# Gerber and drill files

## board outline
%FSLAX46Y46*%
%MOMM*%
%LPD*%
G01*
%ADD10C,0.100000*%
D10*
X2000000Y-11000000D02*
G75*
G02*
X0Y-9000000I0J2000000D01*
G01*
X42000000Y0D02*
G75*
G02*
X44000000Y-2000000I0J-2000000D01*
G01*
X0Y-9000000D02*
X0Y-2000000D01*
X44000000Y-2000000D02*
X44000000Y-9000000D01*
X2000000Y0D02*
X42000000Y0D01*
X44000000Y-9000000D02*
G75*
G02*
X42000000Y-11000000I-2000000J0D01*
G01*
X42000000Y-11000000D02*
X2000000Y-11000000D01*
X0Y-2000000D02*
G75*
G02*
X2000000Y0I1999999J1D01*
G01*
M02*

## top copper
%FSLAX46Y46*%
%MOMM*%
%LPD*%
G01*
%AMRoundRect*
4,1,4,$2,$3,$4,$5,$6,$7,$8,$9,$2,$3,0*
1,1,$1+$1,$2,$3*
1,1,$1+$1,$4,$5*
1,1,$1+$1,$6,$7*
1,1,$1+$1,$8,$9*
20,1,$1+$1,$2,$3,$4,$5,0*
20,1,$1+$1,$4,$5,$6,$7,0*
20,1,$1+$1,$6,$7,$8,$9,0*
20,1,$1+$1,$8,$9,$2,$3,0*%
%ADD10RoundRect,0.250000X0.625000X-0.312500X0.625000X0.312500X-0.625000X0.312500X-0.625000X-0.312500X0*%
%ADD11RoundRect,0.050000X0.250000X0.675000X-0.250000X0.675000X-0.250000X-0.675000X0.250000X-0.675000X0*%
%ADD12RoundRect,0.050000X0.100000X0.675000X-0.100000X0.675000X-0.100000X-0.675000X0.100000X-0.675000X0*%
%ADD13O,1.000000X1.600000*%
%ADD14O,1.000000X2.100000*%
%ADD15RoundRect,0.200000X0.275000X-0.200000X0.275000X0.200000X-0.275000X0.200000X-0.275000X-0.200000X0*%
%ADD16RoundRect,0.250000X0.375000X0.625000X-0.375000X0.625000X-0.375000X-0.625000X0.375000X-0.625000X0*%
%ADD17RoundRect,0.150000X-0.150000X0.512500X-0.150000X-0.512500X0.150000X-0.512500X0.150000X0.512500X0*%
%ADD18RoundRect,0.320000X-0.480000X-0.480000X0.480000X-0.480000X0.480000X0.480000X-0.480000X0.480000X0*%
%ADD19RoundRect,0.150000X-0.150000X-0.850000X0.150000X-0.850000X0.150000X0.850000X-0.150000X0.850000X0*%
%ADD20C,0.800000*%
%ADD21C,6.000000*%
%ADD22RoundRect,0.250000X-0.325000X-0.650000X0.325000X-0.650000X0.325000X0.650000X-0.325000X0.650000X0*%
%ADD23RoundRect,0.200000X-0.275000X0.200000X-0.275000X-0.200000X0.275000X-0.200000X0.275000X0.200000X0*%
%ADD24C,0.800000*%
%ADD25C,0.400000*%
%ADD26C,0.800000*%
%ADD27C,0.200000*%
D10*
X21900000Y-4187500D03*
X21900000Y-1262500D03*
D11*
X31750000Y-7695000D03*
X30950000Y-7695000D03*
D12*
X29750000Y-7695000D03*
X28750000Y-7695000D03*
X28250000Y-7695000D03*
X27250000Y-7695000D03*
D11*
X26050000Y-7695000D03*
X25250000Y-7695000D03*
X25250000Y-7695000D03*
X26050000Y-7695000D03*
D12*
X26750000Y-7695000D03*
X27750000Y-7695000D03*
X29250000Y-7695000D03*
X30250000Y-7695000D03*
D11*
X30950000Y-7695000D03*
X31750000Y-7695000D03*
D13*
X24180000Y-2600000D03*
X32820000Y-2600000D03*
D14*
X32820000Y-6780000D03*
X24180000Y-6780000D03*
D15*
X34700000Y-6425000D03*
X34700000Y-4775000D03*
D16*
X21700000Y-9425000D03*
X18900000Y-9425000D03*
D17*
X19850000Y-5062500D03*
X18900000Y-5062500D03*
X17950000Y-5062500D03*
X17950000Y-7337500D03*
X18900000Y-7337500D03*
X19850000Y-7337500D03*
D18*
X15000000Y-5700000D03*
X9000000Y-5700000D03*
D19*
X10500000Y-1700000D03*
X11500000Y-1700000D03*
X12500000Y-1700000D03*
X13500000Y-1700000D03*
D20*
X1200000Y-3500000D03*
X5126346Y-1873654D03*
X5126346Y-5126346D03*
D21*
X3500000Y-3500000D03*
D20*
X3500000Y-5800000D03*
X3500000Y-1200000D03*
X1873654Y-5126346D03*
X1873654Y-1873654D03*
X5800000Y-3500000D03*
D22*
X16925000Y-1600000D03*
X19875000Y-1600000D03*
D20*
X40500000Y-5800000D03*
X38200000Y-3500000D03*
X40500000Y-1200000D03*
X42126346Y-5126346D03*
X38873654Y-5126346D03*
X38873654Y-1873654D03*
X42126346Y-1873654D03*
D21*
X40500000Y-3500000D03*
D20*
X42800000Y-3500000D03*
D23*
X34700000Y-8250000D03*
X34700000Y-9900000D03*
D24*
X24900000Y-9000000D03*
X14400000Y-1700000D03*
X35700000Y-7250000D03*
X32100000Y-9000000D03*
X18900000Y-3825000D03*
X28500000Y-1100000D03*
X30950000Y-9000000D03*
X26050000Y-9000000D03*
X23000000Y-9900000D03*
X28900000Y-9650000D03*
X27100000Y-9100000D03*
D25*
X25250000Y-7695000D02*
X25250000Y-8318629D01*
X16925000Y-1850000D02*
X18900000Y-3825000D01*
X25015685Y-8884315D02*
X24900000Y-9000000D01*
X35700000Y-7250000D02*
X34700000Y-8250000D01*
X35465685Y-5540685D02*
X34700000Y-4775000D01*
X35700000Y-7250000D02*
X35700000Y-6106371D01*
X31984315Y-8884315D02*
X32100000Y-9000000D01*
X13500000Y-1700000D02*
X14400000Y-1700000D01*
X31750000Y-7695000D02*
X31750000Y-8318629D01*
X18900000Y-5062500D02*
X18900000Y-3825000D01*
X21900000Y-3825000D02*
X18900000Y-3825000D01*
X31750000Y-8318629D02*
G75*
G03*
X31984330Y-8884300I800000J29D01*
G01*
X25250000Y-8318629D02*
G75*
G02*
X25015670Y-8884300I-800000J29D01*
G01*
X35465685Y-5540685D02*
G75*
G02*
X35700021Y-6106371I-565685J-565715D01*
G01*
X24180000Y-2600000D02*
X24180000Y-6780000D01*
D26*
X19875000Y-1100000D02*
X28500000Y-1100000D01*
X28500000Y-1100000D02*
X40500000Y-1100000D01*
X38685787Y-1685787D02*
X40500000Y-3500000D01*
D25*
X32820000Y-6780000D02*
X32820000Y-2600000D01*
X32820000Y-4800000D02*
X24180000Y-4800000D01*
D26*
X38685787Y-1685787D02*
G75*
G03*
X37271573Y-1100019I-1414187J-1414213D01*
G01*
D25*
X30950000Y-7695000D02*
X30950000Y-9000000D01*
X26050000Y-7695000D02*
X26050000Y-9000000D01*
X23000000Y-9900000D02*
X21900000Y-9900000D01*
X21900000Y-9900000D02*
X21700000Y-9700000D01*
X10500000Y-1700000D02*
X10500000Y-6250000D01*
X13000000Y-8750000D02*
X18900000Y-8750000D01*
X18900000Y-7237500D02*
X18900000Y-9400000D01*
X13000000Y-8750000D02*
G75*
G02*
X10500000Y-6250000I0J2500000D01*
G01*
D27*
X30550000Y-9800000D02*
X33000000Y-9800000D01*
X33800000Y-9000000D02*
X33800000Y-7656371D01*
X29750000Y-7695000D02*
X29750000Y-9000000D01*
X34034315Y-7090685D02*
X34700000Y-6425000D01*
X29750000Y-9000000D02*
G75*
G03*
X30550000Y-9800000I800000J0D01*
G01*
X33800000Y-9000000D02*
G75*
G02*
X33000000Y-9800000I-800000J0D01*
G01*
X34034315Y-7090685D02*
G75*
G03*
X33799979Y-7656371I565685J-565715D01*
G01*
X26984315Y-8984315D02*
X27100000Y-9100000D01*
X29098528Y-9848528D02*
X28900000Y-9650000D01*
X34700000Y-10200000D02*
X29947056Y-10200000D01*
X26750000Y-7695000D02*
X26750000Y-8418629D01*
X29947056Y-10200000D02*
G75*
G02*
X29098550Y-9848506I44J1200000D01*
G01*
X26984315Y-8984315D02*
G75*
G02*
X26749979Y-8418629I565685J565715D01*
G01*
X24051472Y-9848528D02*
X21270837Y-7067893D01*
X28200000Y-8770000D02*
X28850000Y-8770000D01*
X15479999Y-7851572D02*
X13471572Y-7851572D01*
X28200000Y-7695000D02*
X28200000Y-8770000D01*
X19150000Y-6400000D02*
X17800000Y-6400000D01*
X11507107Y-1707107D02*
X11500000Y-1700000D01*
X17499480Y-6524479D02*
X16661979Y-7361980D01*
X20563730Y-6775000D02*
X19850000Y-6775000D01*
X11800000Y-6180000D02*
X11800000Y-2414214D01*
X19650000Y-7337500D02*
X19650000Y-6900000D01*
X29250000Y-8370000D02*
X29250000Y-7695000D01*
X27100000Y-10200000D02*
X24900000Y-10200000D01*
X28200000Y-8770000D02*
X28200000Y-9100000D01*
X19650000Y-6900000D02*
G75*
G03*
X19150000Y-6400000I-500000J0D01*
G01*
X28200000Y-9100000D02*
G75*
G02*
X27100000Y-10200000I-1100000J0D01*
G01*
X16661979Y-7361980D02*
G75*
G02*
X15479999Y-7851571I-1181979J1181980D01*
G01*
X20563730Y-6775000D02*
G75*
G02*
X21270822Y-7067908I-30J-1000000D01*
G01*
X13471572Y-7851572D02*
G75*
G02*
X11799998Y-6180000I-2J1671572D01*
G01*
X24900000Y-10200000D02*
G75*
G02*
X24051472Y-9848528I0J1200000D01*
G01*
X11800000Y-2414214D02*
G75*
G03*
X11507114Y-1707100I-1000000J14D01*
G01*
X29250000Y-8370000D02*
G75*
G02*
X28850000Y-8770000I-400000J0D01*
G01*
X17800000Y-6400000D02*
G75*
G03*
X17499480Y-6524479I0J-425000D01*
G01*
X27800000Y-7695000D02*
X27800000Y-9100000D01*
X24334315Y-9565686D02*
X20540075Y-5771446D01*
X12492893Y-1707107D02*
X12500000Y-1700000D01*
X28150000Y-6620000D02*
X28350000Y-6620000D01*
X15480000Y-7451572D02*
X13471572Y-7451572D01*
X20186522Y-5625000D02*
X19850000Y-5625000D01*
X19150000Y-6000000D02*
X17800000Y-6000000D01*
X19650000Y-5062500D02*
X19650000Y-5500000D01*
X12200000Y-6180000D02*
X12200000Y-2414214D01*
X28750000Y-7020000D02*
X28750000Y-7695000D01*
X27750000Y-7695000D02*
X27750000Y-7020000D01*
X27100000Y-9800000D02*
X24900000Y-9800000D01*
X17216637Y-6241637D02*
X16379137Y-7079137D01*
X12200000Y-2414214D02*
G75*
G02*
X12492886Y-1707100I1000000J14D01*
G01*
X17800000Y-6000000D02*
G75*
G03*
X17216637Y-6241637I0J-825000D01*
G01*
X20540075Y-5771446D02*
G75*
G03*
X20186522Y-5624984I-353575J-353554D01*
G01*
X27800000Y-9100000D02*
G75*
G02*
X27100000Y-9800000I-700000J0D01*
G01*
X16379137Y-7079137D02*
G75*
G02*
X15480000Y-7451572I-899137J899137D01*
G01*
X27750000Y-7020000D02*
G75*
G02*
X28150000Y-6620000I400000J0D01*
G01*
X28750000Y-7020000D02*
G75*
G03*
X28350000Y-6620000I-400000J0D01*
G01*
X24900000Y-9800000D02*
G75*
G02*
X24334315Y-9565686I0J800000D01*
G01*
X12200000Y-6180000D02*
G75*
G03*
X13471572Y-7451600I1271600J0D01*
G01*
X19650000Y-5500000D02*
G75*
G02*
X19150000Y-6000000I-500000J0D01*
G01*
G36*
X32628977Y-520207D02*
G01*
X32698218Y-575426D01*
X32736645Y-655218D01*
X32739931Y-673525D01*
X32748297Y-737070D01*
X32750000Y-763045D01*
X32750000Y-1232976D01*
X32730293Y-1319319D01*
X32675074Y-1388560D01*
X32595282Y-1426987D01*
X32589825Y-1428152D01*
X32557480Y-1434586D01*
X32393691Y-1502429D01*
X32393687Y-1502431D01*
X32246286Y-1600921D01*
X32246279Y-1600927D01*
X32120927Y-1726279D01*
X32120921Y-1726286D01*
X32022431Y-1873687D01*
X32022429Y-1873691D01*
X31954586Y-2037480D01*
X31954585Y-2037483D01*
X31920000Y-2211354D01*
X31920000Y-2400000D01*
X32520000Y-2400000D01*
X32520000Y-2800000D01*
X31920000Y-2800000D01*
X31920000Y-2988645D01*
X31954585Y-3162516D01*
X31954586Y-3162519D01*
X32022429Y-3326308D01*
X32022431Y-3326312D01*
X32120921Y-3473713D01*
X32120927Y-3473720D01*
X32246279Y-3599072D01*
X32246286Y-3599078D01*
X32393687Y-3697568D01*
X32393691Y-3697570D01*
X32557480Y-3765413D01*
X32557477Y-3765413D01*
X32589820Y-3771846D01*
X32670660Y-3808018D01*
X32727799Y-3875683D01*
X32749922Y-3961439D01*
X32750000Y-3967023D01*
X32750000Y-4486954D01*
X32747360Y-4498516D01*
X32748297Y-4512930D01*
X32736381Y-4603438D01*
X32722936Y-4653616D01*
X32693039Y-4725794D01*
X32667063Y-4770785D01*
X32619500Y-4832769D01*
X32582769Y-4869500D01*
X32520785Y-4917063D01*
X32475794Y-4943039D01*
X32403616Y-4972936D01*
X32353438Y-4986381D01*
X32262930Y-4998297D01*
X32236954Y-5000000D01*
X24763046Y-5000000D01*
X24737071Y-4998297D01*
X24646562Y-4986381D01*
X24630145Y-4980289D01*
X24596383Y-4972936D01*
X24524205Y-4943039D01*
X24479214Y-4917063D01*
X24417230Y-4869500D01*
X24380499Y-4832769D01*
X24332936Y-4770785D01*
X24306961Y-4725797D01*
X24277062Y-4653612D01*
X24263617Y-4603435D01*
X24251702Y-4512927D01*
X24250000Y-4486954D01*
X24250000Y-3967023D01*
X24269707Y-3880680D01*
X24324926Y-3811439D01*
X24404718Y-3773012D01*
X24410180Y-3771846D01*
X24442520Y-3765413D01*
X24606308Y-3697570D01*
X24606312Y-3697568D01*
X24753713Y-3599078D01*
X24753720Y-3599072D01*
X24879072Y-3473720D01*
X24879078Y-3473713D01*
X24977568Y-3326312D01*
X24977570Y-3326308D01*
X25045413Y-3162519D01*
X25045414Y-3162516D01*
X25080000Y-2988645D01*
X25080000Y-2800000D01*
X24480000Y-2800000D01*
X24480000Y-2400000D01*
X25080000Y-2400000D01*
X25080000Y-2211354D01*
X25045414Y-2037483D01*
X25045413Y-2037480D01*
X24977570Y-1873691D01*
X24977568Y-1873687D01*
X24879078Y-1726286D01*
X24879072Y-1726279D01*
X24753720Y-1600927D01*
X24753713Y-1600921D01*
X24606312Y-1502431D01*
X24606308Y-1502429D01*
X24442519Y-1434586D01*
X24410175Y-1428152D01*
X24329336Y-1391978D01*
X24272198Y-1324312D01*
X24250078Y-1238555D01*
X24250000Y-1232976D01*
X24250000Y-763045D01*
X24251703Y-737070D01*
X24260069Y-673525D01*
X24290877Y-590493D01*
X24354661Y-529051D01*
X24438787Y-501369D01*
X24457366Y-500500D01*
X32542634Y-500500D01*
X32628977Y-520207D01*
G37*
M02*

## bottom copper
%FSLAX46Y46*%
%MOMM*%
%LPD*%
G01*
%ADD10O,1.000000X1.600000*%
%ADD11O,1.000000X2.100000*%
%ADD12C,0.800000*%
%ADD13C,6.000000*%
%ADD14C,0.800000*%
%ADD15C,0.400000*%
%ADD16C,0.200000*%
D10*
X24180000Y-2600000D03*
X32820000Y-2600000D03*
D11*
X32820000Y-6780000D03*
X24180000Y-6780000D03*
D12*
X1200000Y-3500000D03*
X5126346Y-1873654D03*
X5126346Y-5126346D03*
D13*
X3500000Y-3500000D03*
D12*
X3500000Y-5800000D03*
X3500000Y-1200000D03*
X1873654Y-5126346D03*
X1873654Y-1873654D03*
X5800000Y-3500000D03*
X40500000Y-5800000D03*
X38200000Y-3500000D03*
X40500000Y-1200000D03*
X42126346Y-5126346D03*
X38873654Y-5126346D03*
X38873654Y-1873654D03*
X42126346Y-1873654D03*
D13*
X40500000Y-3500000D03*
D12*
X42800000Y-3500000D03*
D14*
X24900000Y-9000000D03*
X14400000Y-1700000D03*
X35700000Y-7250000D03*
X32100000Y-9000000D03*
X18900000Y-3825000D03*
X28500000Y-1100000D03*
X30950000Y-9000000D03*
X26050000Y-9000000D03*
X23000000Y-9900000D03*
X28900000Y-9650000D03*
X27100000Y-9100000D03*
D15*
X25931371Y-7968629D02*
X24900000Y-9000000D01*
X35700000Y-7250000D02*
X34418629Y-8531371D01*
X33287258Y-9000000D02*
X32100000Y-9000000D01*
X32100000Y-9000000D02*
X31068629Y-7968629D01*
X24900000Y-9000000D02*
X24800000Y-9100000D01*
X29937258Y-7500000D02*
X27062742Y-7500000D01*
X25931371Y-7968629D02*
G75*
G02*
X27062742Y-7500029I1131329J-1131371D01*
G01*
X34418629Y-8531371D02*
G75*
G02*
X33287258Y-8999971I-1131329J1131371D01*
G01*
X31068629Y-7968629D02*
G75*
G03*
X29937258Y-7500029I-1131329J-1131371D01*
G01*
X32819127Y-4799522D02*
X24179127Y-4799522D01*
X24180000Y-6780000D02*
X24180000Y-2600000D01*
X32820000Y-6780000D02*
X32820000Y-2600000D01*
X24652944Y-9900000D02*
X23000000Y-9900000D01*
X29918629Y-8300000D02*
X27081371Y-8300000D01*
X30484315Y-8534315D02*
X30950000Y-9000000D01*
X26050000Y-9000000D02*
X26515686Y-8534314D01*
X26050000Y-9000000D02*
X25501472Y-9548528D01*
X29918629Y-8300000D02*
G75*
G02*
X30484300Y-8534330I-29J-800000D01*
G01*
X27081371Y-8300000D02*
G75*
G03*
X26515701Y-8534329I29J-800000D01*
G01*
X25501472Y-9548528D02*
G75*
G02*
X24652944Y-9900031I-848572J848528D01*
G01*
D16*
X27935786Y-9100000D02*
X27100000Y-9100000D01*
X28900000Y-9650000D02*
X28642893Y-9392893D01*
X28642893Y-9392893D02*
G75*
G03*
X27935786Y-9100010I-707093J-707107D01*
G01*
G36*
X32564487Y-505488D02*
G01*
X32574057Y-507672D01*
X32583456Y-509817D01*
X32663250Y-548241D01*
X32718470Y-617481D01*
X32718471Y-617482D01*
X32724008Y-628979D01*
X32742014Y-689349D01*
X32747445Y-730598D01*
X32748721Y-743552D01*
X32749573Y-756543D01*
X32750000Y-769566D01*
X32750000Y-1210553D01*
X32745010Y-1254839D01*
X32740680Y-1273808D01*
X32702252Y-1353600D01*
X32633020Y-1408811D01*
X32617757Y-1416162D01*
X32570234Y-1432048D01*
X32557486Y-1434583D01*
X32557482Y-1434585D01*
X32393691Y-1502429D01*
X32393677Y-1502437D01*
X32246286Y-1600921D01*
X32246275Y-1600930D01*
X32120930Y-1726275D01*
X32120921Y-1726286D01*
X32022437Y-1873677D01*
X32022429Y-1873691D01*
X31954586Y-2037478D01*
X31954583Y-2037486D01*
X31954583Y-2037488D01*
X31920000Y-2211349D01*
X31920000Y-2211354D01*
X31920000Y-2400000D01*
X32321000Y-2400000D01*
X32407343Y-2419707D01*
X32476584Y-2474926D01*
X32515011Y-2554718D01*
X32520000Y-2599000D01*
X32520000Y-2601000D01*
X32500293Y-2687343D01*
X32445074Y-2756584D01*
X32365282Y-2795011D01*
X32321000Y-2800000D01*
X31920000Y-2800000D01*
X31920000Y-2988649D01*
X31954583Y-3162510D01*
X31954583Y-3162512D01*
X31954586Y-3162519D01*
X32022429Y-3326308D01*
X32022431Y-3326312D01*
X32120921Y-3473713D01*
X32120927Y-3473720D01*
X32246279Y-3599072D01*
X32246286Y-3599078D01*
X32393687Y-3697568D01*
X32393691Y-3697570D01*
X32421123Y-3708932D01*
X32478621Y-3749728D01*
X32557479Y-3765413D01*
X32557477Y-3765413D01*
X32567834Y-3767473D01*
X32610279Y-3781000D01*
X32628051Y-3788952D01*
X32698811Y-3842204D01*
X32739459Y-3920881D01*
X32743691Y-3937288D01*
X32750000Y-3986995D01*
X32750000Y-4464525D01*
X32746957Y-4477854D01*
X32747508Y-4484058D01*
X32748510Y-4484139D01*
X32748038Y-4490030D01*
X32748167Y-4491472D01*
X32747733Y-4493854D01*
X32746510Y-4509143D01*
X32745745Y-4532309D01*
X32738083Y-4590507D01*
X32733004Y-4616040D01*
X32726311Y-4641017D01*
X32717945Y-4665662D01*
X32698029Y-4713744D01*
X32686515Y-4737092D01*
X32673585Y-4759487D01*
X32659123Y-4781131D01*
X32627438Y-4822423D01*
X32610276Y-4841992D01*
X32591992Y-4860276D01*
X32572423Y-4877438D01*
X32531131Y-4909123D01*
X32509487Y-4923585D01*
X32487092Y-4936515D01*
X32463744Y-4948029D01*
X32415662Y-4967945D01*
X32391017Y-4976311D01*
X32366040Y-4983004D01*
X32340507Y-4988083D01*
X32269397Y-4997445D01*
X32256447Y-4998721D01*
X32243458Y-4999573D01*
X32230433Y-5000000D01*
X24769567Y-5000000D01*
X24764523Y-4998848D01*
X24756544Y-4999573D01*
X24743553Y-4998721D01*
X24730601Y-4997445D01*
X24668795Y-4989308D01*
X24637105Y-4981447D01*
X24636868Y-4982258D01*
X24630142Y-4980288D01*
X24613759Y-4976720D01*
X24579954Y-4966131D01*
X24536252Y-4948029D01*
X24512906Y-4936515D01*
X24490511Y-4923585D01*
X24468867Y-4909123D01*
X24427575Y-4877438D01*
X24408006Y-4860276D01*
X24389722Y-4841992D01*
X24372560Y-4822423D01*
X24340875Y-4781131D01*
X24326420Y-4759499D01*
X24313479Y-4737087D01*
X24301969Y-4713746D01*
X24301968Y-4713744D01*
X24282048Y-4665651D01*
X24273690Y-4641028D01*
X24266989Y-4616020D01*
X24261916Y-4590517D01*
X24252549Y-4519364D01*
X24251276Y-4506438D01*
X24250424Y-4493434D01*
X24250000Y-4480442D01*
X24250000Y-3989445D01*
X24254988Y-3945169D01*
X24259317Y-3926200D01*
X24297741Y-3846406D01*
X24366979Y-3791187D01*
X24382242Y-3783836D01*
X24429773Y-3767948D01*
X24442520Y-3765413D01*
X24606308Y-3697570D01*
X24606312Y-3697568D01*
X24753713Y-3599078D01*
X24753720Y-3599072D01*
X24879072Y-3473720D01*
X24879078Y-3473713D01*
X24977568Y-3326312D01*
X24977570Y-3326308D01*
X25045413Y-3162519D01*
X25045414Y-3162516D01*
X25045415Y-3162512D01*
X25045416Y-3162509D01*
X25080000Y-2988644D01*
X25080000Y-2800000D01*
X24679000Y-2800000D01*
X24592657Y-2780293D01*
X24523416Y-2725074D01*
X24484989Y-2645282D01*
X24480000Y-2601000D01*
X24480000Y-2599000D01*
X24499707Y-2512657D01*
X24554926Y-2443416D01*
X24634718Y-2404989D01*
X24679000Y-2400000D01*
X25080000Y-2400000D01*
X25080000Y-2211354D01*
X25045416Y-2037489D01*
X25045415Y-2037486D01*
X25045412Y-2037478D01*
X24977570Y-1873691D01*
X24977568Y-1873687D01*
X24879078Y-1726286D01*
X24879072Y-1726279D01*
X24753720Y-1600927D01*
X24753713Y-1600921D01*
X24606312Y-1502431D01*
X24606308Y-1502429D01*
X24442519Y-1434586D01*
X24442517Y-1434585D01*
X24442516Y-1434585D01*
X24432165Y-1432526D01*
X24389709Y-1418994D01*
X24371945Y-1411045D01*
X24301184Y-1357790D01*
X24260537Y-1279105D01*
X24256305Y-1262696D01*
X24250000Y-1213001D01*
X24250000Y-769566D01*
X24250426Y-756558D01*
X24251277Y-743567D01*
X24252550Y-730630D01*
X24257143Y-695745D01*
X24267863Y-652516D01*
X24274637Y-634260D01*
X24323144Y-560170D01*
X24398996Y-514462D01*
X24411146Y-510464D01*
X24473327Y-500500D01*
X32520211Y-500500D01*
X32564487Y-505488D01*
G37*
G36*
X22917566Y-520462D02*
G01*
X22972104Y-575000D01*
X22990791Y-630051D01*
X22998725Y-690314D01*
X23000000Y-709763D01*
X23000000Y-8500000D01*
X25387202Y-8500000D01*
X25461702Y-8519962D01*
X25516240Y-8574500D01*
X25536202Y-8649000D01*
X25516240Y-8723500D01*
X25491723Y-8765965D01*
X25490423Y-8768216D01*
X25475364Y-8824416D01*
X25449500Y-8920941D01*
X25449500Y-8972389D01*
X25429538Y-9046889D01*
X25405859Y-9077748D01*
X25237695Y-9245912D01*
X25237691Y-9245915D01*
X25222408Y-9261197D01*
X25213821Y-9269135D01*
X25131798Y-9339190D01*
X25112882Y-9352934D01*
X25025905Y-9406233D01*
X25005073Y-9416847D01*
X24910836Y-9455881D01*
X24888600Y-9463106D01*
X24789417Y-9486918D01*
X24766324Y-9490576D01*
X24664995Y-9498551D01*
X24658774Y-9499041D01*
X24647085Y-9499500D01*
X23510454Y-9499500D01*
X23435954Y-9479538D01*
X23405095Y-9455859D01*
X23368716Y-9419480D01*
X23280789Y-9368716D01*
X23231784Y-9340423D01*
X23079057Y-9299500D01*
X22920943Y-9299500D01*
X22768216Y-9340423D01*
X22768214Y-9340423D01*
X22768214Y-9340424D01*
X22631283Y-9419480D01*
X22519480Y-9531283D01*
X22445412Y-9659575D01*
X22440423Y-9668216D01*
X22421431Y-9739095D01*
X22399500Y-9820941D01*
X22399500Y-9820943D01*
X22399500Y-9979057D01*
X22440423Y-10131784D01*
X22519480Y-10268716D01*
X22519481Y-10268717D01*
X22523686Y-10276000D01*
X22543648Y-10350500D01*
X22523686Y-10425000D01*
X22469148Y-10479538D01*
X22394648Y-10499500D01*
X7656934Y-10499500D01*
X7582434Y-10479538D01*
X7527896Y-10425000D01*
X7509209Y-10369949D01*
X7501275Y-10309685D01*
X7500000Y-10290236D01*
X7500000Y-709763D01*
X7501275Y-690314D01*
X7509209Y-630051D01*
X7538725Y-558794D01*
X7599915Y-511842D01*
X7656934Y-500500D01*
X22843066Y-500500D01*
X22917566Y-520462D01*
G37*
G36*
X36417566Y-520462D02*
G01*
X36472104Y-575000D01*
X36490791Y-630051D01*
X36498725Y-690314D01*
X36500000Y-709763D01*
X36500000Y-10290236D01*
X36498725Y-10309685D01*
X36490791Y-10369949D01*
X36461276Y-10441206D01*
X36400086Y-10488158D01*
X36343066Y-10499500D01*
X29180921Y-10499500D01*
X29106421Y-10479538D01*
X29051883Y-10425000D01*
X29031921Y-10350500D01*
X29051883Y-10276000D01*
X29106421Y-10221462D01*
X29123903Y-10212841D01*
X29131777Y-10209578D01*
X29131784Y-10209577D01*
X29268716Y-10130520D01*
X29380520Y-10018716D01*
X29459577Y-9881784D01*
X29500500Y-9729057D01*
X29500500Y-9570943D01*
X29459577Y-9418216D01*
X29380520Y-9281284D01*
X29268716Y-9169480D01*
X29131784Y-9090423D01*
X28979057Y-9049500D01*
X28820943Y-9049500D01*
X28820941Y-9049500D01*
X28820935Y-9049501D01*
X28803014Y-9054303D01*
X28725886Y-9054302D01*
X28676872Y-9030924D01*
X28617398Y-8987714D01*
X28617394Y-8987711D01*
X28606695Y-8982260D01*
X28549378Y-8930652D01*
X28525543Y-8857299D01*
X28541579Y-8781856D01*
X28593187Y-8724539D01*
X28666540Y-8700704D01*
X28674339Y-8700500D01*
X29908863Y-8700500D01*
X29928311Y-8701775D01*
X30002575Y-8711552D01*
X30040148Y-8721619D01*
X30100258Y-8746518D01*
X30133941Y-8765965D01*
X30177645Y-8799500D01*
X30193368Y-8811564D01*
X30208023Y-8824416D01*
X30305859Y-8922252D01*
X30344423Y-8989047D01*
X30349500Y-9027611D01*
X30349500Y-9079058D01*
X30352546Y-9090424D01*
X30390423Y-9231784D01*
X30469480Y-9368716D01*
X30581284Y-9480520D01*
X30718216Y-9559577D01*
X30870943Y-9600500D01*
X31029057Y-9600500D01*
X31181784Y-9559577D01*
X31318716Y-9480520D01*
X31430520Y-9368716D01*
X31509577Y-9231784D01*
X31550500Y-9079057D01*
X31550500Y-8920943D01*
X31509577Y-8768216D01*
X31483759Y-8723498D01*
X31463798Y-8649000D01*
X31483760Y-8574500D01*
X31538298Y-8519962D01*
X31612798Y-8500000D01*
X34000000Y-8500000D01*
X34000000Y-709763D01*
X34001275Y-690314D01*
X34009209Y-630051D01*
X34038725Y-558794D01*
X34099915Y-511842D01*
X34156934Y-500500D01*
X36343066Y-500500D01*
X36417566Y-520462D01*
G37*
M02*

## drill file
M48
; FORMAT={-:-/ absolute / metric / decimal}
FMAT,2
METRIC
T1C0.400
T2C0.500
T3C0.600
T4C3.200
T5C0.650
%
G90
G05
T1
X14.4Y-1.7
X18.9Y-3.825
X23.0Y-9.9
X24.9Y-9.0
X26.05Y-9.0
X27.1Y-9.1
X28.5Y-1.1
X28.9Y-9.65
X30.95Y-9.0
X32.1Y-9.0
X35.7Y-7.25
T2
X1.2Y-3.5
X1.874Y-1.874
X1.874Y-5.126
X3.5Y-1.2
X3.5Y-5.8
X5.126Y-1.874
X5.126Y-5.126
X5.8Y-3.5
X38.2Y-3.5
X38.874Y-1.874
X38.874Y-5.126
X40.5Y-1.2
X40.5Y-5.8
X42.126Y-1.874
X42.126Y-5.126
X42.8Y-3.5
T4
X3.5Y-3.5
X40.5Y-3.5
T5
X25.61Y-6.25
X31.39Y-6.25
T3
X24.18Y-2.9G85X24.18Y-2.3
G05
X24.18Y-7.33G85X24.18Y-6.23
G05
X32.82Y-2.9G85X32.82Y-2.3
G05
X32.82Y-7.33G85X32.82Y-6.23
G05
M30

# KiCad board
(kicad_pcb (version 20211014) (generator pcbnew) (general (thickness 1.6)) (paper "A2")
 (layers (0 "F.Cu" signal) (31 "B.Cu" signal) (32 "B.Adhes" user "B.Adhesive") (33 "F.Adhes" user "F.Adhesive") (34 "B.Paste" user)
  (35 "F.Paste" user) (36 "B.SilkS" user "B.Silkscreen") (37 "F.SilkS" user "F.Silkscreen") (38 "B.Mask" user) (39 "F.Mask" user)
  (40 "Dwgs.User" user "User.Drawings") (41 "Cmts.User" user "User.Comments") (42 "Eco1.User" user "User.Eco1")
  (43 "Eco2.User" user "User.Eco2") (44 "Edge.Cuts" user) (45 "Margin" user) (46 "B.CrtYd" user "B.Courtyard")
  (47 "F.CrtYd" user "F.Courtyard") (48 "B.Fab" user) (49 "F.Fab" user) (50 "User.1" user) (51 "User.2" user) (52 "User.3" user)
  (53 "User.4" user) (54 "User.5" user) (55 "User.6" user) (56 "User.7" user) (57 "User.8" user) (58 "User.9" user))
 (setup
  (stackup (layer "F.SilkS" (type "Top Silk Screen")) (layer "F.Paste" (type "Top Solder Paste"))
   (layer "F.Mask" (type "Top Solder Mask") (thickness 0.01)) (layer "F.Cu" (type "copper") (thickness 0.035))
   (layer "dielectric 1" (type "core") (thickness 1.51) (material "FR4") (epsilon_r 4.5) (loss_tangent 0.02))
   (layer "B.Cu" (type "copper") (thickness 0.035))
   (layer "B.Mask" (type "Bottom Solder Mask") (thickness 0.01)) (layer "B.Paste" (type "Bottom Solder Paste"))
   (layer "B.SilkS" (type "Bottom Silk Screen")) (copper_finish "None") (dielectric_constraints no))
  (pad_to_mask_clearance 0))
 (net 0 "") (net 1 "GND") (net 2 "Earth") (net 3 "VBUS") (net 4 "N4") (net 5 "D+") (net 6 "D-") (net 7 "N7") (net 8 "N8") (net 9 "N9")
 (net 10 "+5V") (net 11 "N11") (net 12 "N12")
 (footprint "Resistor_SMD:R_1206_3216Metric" (layer "F.Cu") (at 21.9 2.725 90)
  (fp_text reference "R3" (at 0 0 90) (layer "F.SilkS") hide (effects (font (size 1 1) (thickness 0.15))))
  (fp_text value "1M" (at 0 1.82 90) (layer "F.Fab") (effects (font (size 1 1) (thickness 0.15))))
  (pad "1" smd roundrect (at -1.4625 0 90) (size 1.125 1.75) (layers "F.Cu" "F.Paste" "F.Mask") (roundrect_rratio 0.2222222222)
   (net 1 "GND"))
  (pad "2" smd roundrect (at 1.4625 0 90) (size 1.125 1.75) (layers "F.Cu" "F.Paste" "F.Mask") (roundrect_rratio 0.2222222222)
   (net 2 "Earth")))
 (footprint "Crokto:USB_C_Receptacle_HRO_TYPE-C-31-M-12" (layer "F.Cu") (at 28.5 3.65 180)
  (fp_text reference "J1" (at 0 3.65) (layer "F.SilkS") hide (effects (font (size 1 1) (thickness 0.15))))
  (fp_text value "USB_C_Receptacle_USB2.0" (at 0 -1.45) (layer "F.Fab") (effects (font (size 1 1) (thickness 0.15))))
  (pad "" np_thru_hole circle (at -2.89 -2.6 180) (size 0.65 0.65) (drill 0.65) (layers *.Cu *.Mask))
  (pad "" np_thru_hole circle (at 2.89 -2.6 180) (size 0.65 0.65) (drill 0.65) (layers *.Cu *.Mask))
  (pad "A1" smd roundrect (at -3.25 -4.045 180) (size 0.6 1.45) (layers "F.Cu" "F.Paste" "F.Mask") (roundrect_rratio 0.08333333333)
   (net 1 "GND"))
  (pad "A4" smd roundrect (at -2.45 -4.045 180) (size 0.6 1.45) (layers "F.Cu" "F.Paste" "F.Mask") (roundrect_rratio 0.08333333333)
   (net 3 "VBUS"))
  (pad "A5" smd roundrect (at -1.25 -4.045 180) (size 0.3 1.45) (layers "F.Cu" "F.Paste" "F.Mask") (roundrect_rratio 0.1666666667)
   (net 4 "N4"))
  (pad "A6" smd roundrect (at -0.25 -4.045 180) (size 0.3 1.45) (layers "F.Cu" "F.Paste" "F.Mask") (roundrect_rratio 0.1666666667)
   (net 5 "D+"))
  (pad "A7" smd roundrect (at 0.25 -4.045 180) (size 0.3 1.45) (layers "F.Cu" "F.Paste" "F.Mask") (roundrect_rratio 0.1666666667)
   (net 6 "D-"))
  (pad "A8" smd roundrect (at 1.25 -4.045 180) (size 0.3 1.45) (layers "F.Cu" "F.Paste" "F.Mask") (roundrect_rratio 0.1666666667)
   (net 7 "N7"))
  (pad "A9" smd roundrect (at 2.45 -4.045 180) (size 0.6 1.45) (layers "F.Cu" "F.Paste" "F.Mask") (roundrect_rratio 0.08333333333)
   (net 3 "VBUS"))
  (pad "A12" smd roundrect (at 3.25 -4.045 180) (size 0.6 1.45) (layers "F.Cu" "F.Paste" "F.Mask") (roundrect_rratio 0.08333333333)
   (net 1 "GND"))
  (pad "B1" smd roundrect (at 3.25 -4.045 180) (size 0.6 1.45) (layers "F.Cu" "F.Paste" "F.Mask") (roundrect_rratio 0.08333333333)
   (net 1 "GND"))
  (pad "B4" smd roundrect (at 2.45 -4.045 180) (size 0.6 1.45) (layers "F.Cu" "F.Paste" "F.Mask") (roundrect_rratio 0.08333333333)
   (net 3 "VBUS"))
  (pad "B5" smd roundrect (at 1.75 -4.045 180) (size 0.3 1.45) (layers "F.Cu" "F.Paste" "F.Mask") (roundrect_rratio 0.1666666667)
   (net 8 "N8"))
  (pad "B6" smd roundrect (at 0.75 -4.045 180) (size 0.3 1.45) (layers "F.Cu" "F.Paste" "F.Mask") (roundrect_rratio 0.1666666667)
   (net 5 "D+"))
  (pad "B7" smd roundrect (at -0.75 -4.045 180) (size 0.3 1.45) (layers "F.Cu" "F.Paste" "F.Mask") (roundrect_rratio 0.1666666667)
   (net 6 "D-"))
  (pad "B8" smd roundrect (at -1.75 -4.045 180) (size 0.3 1.45) (layers "F.Cu" "F.Paste" "F.Mask") (roundrect_rratio 0.1666666667)
   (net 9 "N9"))
  (pad "B9" smd roundrect (at -2.45 -4.045 180) (size 0.6 1.45) (layers "F.Cu" "F.Paste" "F.Mask") (roundrect_rratio 0.08333333333)
   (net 3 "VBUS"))
  (pad "B12" smd roundrect (at -3.25 -4.045 180) (size 0.6 1.45) (layers "F.Cu" "F.Paste" "F.Mask") (roundrect_rratio 0.08333333333)
   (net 1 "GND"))
  (pad "S1" thru_hole oval (at 4.32 1.05 180) (size 1 1.6) (drill oval 0.6 1.2) (layers *.Cu *.Mask) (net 2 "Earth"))
  (pad "S1" thru_hole oval (at -4.32 1.05 180) (size 1 1.6) (drill oval 0.6 1.2) (layers *.Cu *.Mask) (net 2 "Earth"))
  (pad "S1" thru_hole oval (at -4.32 -3.13 180) (size 1 2.1) (drill oval 0.6 1.7) (layers *.Cu *.Mask) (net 2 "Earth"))
  (pad "S1" thru_hole oval (at 4.32 -3.13 180) (size 1 2.1) (drill oval 0.6 1.7) (layers *.Cu *.Mask) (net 2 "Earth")))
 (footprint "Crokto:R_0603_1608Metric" (layer "F.Cu") (at 34.7 5.6 90)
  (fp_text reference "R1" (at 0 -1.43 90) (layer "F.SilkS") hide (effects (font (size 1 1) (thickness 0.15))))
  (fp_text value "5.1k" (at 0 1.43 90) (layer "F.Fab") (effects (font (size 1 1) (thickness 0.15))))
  (pad "1" smd roundrect (at -0.825 0 90) (size 0.8 0.95) (layers "F.Cu" "F.Paste" "F.Mask") (roundrect_rratio 0.25) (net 4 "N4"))
  (pad "2" smd roundrect (at 0.825 0 90) (size 0.8 0.95) (layers "F.Cu" "F.Paste" "F.Mask") (roundrect_rratio 0.25) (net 1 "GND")))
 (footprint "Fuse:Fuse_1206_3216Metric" (layer "F.Cu") (at 20.3 9.425 180)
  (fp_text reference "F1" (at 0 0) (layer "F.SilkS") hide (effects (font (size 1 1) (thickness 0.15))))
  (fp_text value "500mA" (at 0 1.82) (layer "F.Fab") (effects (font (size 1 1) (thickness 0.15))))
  (pad "1" smd roundrect (at -1.4 0 180) (size 1.25 1.75) (layers "F.Cu" "F.Paste" "F.Mask") (roundrect_rratio 0.2) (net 3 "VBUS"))
  (pad "2" smd roundrect (at 1.4 0 180) (size 1.25 1.75) (layers "F.Cu" "F.Paste" "F.Mask") (roundrect_rratio 0.2) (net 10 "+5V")))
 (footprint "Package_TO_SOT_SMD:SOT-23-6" (layer "F.Cu") (at 18.9 6.2 -90)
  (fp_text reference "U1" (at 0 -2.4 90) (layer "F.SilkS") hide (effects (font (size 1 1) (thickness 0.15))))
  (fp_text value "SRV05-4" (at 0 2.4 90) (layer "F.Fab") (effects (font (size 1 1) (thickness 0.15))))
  (pad "1" smd roundrect (at -1.1375 -0.95 270) (size 1.325 0.6) (layers "F.Cu" "F.Paste" "F.Mask") (roundrect_rratio 0.25) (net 5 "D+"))
  (pad "2" smd roundrect (at -1.1375 0 270) (size 1.325 0.6) (layers "F.Cu" "F.Paste" "F.Mask") (roundrect_rratio 0.25) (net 1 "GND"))
  (pad "3" smd roundrect (at -1.1375 0.95 270) (size 1.325 0.6) (layers "F.Cu" "F.Paste" "F.Mask") (roundrect_rratio 0.25) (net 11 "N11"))
  (pad "4" smd roundrect (at 1.1375 0.95 270) (size 1.325 0.6) (layers "F.Cu" "F.Paste" "F.Mask") (roundrect_rratio 0.25) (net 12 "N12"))
  (pad "5" smd roundrect (at 1.1375 0 270) (size 1.325 0.6) (layers "F.Cu" "F.Paste" "F.Mask") (roundrect_rratio 0.25) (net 10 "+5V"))
  (pad "6" smd roundrect (at 1.1375 -0.95 270) (size 1.325 0.6) (layers "F.Cu" "F.Paste" "F.Mask") (roundrect_rratio 0.25) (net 6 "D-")))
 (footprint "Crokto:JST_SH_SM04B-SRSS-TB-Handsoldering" (layer "F.Cu") (at 12 3.925)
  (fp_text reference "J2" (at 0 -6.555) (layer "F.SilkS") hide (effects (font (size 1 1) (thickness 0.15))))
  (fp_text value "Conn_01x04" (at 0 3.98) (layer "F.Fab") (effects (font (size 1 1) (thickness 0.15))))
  (pad "" smd roundrect (at 3 1.775) (size 1.6 1.6) (layers "F.Cu" "F.Paste" "F.Mask") (roundrect_rratio 0.2))
  (pad "" smd roundrect (at -3 1.775) (size 1.6 1.6) (layers "F.Cu" "F.Paste" "F.Mask") (roundrect_rratio 0.2))
  (pad "1" smd roundrect (at -1.5 -2.225) (size 0.6 2) (layers "F.Cu" "F.Paste" "F.Mask") (roundrect_rratio 0.25) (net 10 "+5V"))
  (pad "2" smd roundrect (at -0.5 -2.225) (size 0.6 2) (layers "F.Cu" "F.Paste" "F.Mask") (roundrect_rratio 0.25) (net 6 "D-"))
  (pad "3" smd roundrect (at 0.5 -2.225) (size 0.6 2) (layers "F.Cu" "F.Paste" "F.Mask") (roundrect_rratio 0.25) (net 5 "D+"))
  (pad "4" smd roundrect (at 1.5 -2.225) (size 0.6 2) (layers "F.Cu" "F.Paste" "F.Mask") (roundrect_rratio 0.25) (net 1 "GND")))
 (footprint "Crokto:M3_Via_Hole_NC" (layer "F.Cu") (at 3.5 3.5)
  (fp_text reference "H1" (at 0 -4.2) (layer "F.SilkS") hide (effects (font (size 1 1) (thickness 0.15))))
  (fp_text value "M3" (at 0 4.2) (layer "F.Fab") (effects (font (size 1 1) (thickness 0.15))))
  (pad "" thru_hole circle (at -2.3 0) (size 0.8 0.8) (drill 0.5) (layers *.Cu "F.Mask"))
  (pad "" thru_hole circle (at 1.626346 -1.626346) (size 0.8 0.8) (drill 0.5) (layers *.Cu "F.Mask"))
  (pad "" thru_hole circle (at 1.626346 1.626346) (size 0.8 0.8) (drill 0.5) (layers *.Cu "F.Mask"))
  (pad "" thru_hole circle (at 0 0) (size 6 6) (drill 3.2) (layers *.Cu "F.Mask"))
  (pad "" thru_hole circle (at 0 2.3) (size 0.8 0.8) (drill 0.5) (layers *.Cu "F.Mask"))
  (pad "" thru_hole circle (at 0 -2.3) (size 0.8 0.8) (drill 0.5) (layers *.Cu "F.Mask"))
  (pad "" thru_hole circle (at -1.626346 1.626346) (size 0.8 0.8) (drill 0.5) (layers *.Cu "F.Mask"))
  (pad "" thru_hole circle (at -1.626346 -1.626346) (size 0.8 0.8) (drill 0.5) (layers *.Cu "F.Mask"))
  (pad "" thru_hole circle (at 2.3 0) (size 0.8 0.8) (drill 0.5) (layers *.Cu "F.Mask")))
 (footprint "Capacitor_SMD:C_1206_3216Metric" (layer "F.Cu") (at 18.4 1.6)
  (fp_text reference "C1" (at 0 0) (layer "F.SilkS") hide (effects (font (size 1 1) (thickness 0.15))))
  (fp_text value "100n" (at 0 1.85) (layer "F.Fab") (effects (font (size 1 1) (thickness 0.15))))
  (pad "1" smd roundrect (at -1.475 0) (size 1.15 1.8) (layers "F.Cu" "F.Paste" "F.Mask") (roundrect_rratio 0.2173913043) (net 1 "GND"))
  (pad "2" smd roundrect (at 1.475 0) (size 1.15 1.8) (layers "F.Cu" "F.Paste" "F.Mask") (roundrect_rratio 0.2173913043) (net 2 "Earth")))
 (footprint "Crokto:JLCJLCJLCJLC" (layer "F.Cu") (at 28.5 4.6 180)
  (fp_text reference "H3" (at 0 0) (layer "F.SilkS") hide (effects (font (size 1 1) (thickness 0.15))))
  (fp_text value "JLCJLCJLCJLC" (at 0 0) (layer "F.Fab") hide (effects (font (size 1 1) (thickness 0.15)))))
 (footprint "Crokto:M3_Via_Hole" (layer "F.Cu") (at 40.5 3.5)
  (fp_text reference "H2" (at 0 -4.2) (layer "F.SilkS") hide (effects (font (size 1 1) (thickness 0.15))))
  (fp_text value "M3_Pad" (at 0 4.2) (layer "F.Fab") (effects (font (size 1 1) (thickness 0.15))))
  (pad "1" thru_hole circle locked (at 0 2.3) (size 0.8 0.8) (drill 0.5) (layers *.Cu *.Mask) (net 2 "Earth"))
  (pad "1" thru_hole circle locked (at -2.3 0) (size 0.8 0.8) (drill 0.5) (layers *.Cu *.Mask) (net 2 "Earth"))
  (pad "1" thru_hole circle locked (at 0 -2.3) (size 0.8 0.8) (drill 0.5) (layers *.Cu *.Mask) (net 2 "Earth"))
  (pad "1" thru_hole circle locked (at 1.626346 1.626346) (size 0.8 0.8) (drill 0.5) (layers *.Cu *.Mask) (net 2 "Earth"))
  (pad "1" thru_hole circle locked (at -1.626346 1.626346) (size 0.8 0.8) (drill 0.5) (layers *.Cu *.Mask) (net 2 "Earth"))
  (pad "1" thru_hole circle locked (at -1.626346 -1.626346) (size 0.8 0.8) (drill 0.5) (layers *.Cu *.Mask) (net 2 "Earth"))
  (pad "1" thru_hole circle locked (at 1.626346 -1.626346) (size 0.8 0.8) (drill 0.5) (layers *.Cu *.Mask) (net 2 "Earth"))
  (pad "1" thru_hole circle locked (at 0 0) (size 6 6) (drill 3.2) (layers *.Cu *.Mask) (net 2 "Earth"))
  (pad "1" thru_hole circle locked (at 2.3 0) (size 0.8 0.8) (drill 0.5) (layers *.Cu *.Mask) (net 2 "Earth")))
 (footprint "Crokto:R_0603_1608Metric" (layer "F.Cu") (at 34.7 9.075 -90)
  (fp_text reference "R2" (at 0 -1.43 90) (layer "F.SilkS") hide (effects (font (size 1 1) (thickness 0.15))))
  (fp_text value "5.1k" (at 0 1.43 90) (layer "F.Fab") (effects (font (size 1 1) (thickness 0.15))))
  (pad "1" smd roundrect (at -0.825 0 270) (size 0.8 0.95) (layers "F.Cu" "F.Paste" "F.Mask") (roundrect_rratio 0.25) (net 1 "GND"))
  (pad "2" smd roundrect (at 0.825 0 270) (size 0.8 0.95) (layers "F.Cu" "F.Paste" "F.Mask") (roundrect_rratio 0.25) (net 8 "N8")))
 (gr_arc (start 2 11) (mid 0.585786 10.414214) (end 0 9) (layer "Edge.Cuts") (width 0.1))
 (gr_arc (start 42 0) (mid 43.414214 0.585786) (end 44 2) (layer "Edge.Cuts") (width 0.1))
 (gr_line (start 0 9) (end 0 2) (layer "Edge.Cuts") (width 0.1))
 (gr_line (start 44 2) (end 44 9) (layer "Edge.Cuts") (width 0.1))
 (gr_line (start 2 0) (end 42 0) (layer "Edge.Cuts") (width 0.1))
 (gr_arc (start 44 9) (mid 43.414214 10.414214) (end 42 11) (layer "Edge.Cuts") (width 0.1))
 (gr_line (start 42 11) (end 2 11) (layer "Edge.Cuts") (width 0.1))
 (gr_arc (start 0 2) (mid 0.585786 0.585786) (end 2 0) (layer "Edge.Cuts") (width 0.1))
 (segment (start 25.25 7.695) (end 25.25 8.318629) (width 0.4) (layer "F.Cu") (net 1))
 (segment (start 16.925 1.85) (end 18.9 3.825) (width 0.4) (layer "F.Cu") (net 1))
 (segment (start 25.015685 8.884315) (end 24.9 9) (width 0.4) (layer "F.Cu") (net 1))
 (segment (start 35.7 7.25) (end 34.7 8.25) (width 0.4) (layer "F.Cu") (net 1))
 (segment (start 35.465685 5.540685) (end 34.7 4.775) (width 0.4) (layer "F.Cu") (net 1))
 (segment (start 35.7 7.25) (end 35.7 6.106371) (width 0.4) (layer "F.Cu") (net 1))
 (segment (start 31.984315 8.884315) (end 32.1 9) (width 0.4) (layer "F.Cu") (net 1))
 (segment (start 13.5 1.7) (end 14.4 1.7) (width 0.4) (layer "F.Cu") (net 1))
 (segment (start 31.75 7.695) (end 31.75 8.318629) (width 0.4) (layer "F.Cu") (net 1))
 (segment (start 18.9 5.0625) (end 18.9 3.825) (width 0.4) (layer "F.Cu") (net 1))
 (segment (start 21.9 3.825) (end 18.9 3.825) (width 0.4) (layer "F.Cu") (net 1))
 (via (at 24.9 9) (size 0.8) (drill 0.4) (layers "F.Cu" "B.Cu") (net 1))
 (via (at 14.4 1.7) (size 0.8) (drill 0.4) (layers "F.Cu" "B.Cu") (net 1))
 (via (at 35.7 7.25) (size 0.8) (drill 0.4) (layers "F.Cu" "B.Cu") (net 1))
 (via (at 32.1 9) (size 0.8) (drill 0.4) (layers "F.Cu" "B.Cu") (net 1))
 (via (at 18.9 3.825) (size 0.8) (drill 0.4) (layers "F.Cu" "B.Cu") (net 1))
 (arc (start 31.75 8.318629) (mid 31.810897 8.624776) (end 31.984315 8.884315) (width 0.4) (layer "F.Cu") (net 1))
 (arc (start 25.25 8.318629) (mid 25.189103 8.624776) (end 25.015685 8.884315) (width 0.4) (layer "F.Cu") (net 1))
 (arc (start 35.465685 5.540685) (mid 35.639104 5.800224) (end 35.7 6.106371) (width 0.4) (layer "F.Cu") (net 1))
 (segment (start 25.931371 7.968629) (end 24.9 9) (width 0.4) (layer "B.Cu") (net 1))
 (segment (start 35.7 7.25) (end 34.418629 8.531371) (width 0.4) (layer "B.Cu") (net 1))
 (segment (start 33.287258 9) (end 32.1 9) (width 0.4) (layer "B.Cu") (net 1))
 (segment (start 32.1 9) (end 31.068629 7.968629) (width 0.4) (layer "B.Cu") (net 1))
 (segment (start 24.9 9) (end 24.8 9.1) (width 0.4) (layer "B.Cu") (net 1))
 (segment (start 29.937258 7.5) (end 27.062742 7.5) (width 0.4) (layer "B.Cu") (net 1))
 (arc (start 25.931371 7.968629) (mid 26.450448 7.621793) (end 27.062742 7.5) (width 0.4) (layer "B.Cu") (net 1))
 (arc (start 34.418629 8.531371) (mid 33.899552 8.878207) (end 33.287258 9) (width 0.4) (layer "B.Cu") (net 1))
 (arc (start 31.068629 7.968629) (mid 30.549552 7.621793) (end 29.937258 7.5) (width 0.4) (layer "B.Cu") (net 1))
 (segment (start 24.18 2.6) (end 24.18 6.78) (width 0.4) (layer "F.Cu") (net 2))
 (segment (start 19.875 1.1) (end 28.5 1.1) (width 0.8) (layer "F.Cu") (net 2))
 (segment (start 28.5 1.1) (end 40.5 1.1) (width 0.8) (layer "F.Cu") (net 2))
 (segment (start 38.685787 1.685787) (end 40.5 3.5) (width 0.8) (layer "F.Cu") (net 2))
 (segment (start 32.82 6.78) (end 32.82 2.6) (width 0.4) (layer "F.Cu") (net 2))
 (segment (start 32.82 4.8) (end 24.18 4.8) (width 0.4) (layer "F.Cu") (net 2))
 (via (at 28.5 1.1) (size 0.8) (drill 0.4) (layers "F.Cu" "B.Cu") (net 2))
 (arc (start 38.685787 1.685787) (mid 38.03694 1.252241) (end 37.271573 1.1) (width 0.8) (layer "F.Cu") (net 2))
 (segment (start 32.819127 4.799522) (end 24.179127 4.799522) (width 0.4) (layer "B.Cu") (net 2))
 (segment (start 24.18 6.78) (end 24.18 2.6) (width 0.4) (layer "B.Cu") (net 2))
 (segment (start 32.82 6.78) (end 32.82 2.6) (width 0.4) (layer "B.Cu") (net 2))
 (segment (start 30.95 7.695) (end 30.95 9) (width 0.4) (layer "F.Cu") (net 3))
 (segment (start 26.05 7.695) (end 26.05 9) (width 0.4) (layer "F.Cu") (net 3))
 (segment (start 23 9.9) (end 21.9 9.9) (width 0.4) (layer "F.Cu") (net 3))
 (segment (start 21.9 9.9) (end 21.7 9.7) (width 0.4) (layer "F.Cu") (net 3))
 (via (at 30.95 9) (size 0.8) (drill 0.4) (layers "F.Cu" "B.Cu") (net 3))
 (via (at 26.05 9) (size 0.8) (drill 0.4) (layers "F.Cu" "B.Cu") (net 3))
 (via (at 23 9.9) (size 0.8) (drill 0.4) (layers "F.Cu" "B.Cu") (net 3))
 (segment (start 24.652944 9.9) (end 23 9.9) (width 0.4) (layer "B.Cu") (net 3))
 (segment (start 29.918629 8.3) (end 27.081371 8.3) (width 0.4) (layer "B.Cu") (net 3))
 (segment (start 30.484315 8.534315) (end 30.95 9) (width 0.4) (layer "B.Cu") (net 3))
 (segment (start 26.05 9) (end 26.515686 8.534314) (width 0.4) (layer "B.Cu") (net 3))
 (segment (start 26.05 9) (end 25.501472 9.548528) (width 0.4) (layer "B.Cu") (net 3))
 (arc (start 29.918629 8.3) (mid 30.224776 8.360897) (end 30.484315 8.534315) (width 0.4) (layer "B.Cu") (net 3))
 (arc (start 27.081371 8.3) (mid 26.775225 8.360896) (end 26.515686 8.534314) (width 0.4) (layer "B.Cu") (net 3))
 (arc (start 25.501472 9.548528) (mid 25.112164 9.808655) (end 24.652944 9.9) (width 0.4) (layer "B.Cu") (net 3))
 (segment (start 10.5 1.7) (end 10.5 6.25) (width 0.4) (layer "F.Cu") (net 10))
 (segment (start 13 8.75) (end 18.9 8.75) (width 0.4) (layer "F.Cu") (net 10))
 (segment (start 18.9 7.2375) (end 18.9 9.4) (width 0.4) (layer "F.Cu") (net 10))
 (arc (start 13 8.75) (mid 11.232233 8.017767) (end 10.5 6.25) (width 0.4) (layer "F.Cu") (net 10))
 (segment (start 30.55 9.8) (end 33 9.8) (width 0.2) (layer "F.Cu") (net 4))
 (segment (start 33.8 9) (end 33.8 7.656371) (width 0.2) (layer "F.Cu") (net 4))
 (segment (start 29.75 7.695) (end 29.75 9) (width 0.2) (layer "F.Cu") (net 4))
 (segment (start 34.034315 7.090685) (end 34.7 6.425) (width 0.2) (layer "F.Cu") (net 4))
 (arc (start 29.75 9) (mid 29.984315 9.565685) (end 30.55 9.8) (width 0.2) (layer "F.Cu") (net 4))
 (arc (start 33.8 9) (mid 33.565685 9.565685) (end 33 9.8) (width 0.2) (layer "F.Cu") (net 4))
 (arc (start 34.034315 7.090685) (mid 33.860896 7.350224) (end 33.8 7.656371) (width 0.2) (layer "F.Cu") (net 4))
 (segment (start 26.984315 8.984315) (end 27.1 9.1) (width 0.2) (layer "F.Cu") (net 8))
 (segment (start 29.098528 9.848528) (end 28.9 9.65) (width 0.2) (layer "F.Cu") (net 8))
 (segment (start 34.7 10.2) (end 29.947056 10.2) (width 0.2) (layer "F.Cu") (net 8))
 (segment (start 26.75 7.695) (end 26.75 8.418629) (width 0.2) (layer "F.Cu") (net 8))
 (via (at 28.9 9.65) (size 0.8) (drill 0.4) (layers "F.Cu" "B.Cu") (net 8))
 (via (at 27.1 9.1) (size 0.8) (drill 0.4) (layers "F.Cu" "B.Cu") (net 8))
 (arc (start 29.947056 10.2) (mid 29.487836 10.108655) (end 29.098528 9.848528) (width 0.2) (layer "F.Cu") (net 8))
 (arc (start 26.984315 8.984315) (mid 26.810896 8.724776) (end 26.75 8.418629) (width 0.2) (layer "F.Cu") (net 8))
 (segment (start 27.935786 9.1) (end 27.1 9.1) (width 0.2) (layer "B.Cu") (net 8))
 (segment (start 28.9 9.65) (end 28.642893 9.392893) (width 0.2) (layer "B.Cu") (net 8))
 (arc (start 28.642893 9.392893) (mid 28.31847 9.17612) (end 27.935786 9.1) (width 0.2) (layer "B.Cu") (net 8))
 (segment (start 24.051472 9.848528) (end 21.270837 7.067893) (width 0.2) (layer "F.Cu") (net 6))
 (segment (start 28.2 8.77) (end 28.85 8.77) (width 0.2) (layer "F.Cu") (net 6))
 (segment (start 15.479999 7.851572) (end 13.471572 7.851572) (width 0.2) (layer "F.Cu") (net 6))
 (segment (start 28.2 7.695) (end 28.2 8.77) (width 0.2) (layer "F.Cu") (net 6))
 (segment (start 19.15 6.4) (end 17.8 6.4) (width 0.2) (layer "F.Cu") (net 6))
 (segment (start 11.507107 1.707107) (end 11.5 1.7) (width 0.2) (layer "F.Cu") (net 6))
 (segment (start 17.49948 6.524479) (end 16.661979 7.36198) (width 0.2) (layer "F.Cu") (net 6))
 (segment (start 20.56373 6.775) (end 19.85 6.775) (width 0.2) (layer "F.Cu") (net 6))
 (segment (start 11.8 6.18) (end 11.8 2.414214) (width 0.2) (layer "F.Cu") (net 6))
 (segment (start 19.65 7.3375) (end 19.65 6.9) (width 0.2) (layer "F.Cu") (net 6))
 (segment (start 29.25 8.37) (end 29.25 7.695) (width 0.2) (layer "F.Cu") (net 6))
 (segment (start 27.1 10.2) (end 24.9 10.2) (width 0.2) (layer "F.Cu") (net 6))
 (segment (start 28.2 8.77) (end 28.2 9.1) (width 0.2) (layer "F.Cu") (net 6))
 (arc (start 19.65 6.9) (mid 19.503553 6.546447) (end 19.15 6.4) (width 0.2) (layer "F.Cu") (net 6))
 (arc (start 28.2 9.1) (mid 27.877817 9.877817) (end 27.1 10.2) (width 0.2) (layer "F.Cu") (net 6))
 (arc (start 16.661979 7.36198) (mid 16.119682 7.724331) (end 15.479999 7.851572) (width 0.2) (layer "F.Cu") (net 6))
 (arc (start 20.56373 6.775) (mid 20.946413 6.85112) (end 21.270837 7.067893) (width 0.2) (layer "F.Cu") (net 6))
 (arc (start 13.471572 7.851572) (mid 12.289592 7.36198) (end 11.8 6.18) (width 0.2) (layer "F.Cu") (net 6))
 (arc (start 24.9 10.2) (mid 24.44078 10.108655) (end 24.051472 9.848528) (width 0.2) (layer "F.Cu") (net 6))
 (arc (start 11.8 2.414214) (mid 11.72388 2.031531) (end 11.507107 1.707107) (width 0.2) (layer "F.Cu") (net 6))
 (arc (start 29.25 8.37) (mid 29.132843 8.652843) (end 28.85 8.77) (width 0.2) (layer "F.Cu") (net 6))
 (arc (start 17.8 6.4) (mid 17.63736 6.432351) (end 17.49948 6.524479) (width 0.2) (layer "F.Cu") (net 6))
 (segment (start 27.8 7.695) (end 27.8 9.1) (width 0.2) (layer "F.Cu") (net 5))
 (segment (start 24.334315 9.565686) (end 20.540075 5.771446) (width 0.2) (layer "F.Cu") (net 5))
 (segment (start 12.492893 1.707107) (end 12.5 1.7) (width 0.2) (layer "F.Cu") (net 5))
 (segment (start 28.15 6.62) (end 28.35 6.62) (width 0.2) (layer "F.Cu") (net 5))
 (segment (start 15.48 7.451572) (end 13.471572 7.451572) (width 0.2) (layer "F.Cu") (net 5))
 (segment (start 20.186522 5.625) (end 19.85 5.625) (width 0.2) (layer "F.Cu") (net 5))
 (segment (start 19.15 6) (end 17.8 6) (width 0.2) (layer "F.Cu") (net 5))
 (segment (start 19.65 5.0625) (end 19.65 5.5) (width 0.2) (layer "F.Cu") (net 5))
 (segment (start 12.2 6.18) (end 12.2 2.414214) (width 0.2) (layer "F.Cu") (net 5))
 (segment (start 28.75 7.02) (end 28.75 7.695) (width 0.2) (layer "F.Cu") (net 5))
 (segment (start 27.75 7.695) (end 27.75 7.02) (width 0.2) (layer "F.Cu") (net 5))
 (segment (start 27.1 9.8) (end 24.9 9.8) (width 0.2) (layer "F.Cu") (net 5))
 (segment (start 17.216637 6.241637) (end 16.379137 7.079137) (width 0.2) (layer "F.Cu") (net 5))
 (arc (start 12.2 2.414214) (mid 12.27612 2.031531) (end 12.492893 1.707107) (width 0.2) (layer "F.Cu") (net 5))
 (arc (start 17.8 6) (mid 17.484286 6.0628) (end 17.216637 6.241637) (width 0.2) (layer "F.Cu") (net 5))
 (arc (start 20.540075 5.771446) (mid 20.377863 5.66306) (end 20.186522 5.625) (width 0.2) (layer "F.Cu") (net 5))
 (arc (start 27.8 9.1) (mid 27.594975 9.594975) (end 27.1 9.8) (width 0.2) (layer "F.Cu") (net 5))
 (arc (start 16.379137 7.079137) (mid 15.96661 7.354779) (end 15.48 7.451572) (width 0.2) (layer "F.Cu") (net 5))
 (arc (start 27.75 7.02) (mid 27.867157 6.737157) (end 28.15 6.62) (width 0.2) (layer "F.Cu") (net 5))
 (arc (start 28.75 7.02) (mid 28.632843 6.737157) (end 28.35 6.62) (width 0.2) (layer "F.Cu") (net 5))
 (arc (start 24.9 9.8) (mid 24.593854 9.739104) (end 24.334315 9.565686) (width 0.2) (layer "F.Cu") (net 5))
 (arc (start 12.2 6.18) (mid 12.572435 7.079137) (end 13.471572 7.451572) (width 0.2) (layer "F.Cu") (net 5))
 (arc (start 19.65 5.5) (mid 19.503553 5.853553) (end 19.15 6) (width 0.2) (layer "F.Cu") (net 5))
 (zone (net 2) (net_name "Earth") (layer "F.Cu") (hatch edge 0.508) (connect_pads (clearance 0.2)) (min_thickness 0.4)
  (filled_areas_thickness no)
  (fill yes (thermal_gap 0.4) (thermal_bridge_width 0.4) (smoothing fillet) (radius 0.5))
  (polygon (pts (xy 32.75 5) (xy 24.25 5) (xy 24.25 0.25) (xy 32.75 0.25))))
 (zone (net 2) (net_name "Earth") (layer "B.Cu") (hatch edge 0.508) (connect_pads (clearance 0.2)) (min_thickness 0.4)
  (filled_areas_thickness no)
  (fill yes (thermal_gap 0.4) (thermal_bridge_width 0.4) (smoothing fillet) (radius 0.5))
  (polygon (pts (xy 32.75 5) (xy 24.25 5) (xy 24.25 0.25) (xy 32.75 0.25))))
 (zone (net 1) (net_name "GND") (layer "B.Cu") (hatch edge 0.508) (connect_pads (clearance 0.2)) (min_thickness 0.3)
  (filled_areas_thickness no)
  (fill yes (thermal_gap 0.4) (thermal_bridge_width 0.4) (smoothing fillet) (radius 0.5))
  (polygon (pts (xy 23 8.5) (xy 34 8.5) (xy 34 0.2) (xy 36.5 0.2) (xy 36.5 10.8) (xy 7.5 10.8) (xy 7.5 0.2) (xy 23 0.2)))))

